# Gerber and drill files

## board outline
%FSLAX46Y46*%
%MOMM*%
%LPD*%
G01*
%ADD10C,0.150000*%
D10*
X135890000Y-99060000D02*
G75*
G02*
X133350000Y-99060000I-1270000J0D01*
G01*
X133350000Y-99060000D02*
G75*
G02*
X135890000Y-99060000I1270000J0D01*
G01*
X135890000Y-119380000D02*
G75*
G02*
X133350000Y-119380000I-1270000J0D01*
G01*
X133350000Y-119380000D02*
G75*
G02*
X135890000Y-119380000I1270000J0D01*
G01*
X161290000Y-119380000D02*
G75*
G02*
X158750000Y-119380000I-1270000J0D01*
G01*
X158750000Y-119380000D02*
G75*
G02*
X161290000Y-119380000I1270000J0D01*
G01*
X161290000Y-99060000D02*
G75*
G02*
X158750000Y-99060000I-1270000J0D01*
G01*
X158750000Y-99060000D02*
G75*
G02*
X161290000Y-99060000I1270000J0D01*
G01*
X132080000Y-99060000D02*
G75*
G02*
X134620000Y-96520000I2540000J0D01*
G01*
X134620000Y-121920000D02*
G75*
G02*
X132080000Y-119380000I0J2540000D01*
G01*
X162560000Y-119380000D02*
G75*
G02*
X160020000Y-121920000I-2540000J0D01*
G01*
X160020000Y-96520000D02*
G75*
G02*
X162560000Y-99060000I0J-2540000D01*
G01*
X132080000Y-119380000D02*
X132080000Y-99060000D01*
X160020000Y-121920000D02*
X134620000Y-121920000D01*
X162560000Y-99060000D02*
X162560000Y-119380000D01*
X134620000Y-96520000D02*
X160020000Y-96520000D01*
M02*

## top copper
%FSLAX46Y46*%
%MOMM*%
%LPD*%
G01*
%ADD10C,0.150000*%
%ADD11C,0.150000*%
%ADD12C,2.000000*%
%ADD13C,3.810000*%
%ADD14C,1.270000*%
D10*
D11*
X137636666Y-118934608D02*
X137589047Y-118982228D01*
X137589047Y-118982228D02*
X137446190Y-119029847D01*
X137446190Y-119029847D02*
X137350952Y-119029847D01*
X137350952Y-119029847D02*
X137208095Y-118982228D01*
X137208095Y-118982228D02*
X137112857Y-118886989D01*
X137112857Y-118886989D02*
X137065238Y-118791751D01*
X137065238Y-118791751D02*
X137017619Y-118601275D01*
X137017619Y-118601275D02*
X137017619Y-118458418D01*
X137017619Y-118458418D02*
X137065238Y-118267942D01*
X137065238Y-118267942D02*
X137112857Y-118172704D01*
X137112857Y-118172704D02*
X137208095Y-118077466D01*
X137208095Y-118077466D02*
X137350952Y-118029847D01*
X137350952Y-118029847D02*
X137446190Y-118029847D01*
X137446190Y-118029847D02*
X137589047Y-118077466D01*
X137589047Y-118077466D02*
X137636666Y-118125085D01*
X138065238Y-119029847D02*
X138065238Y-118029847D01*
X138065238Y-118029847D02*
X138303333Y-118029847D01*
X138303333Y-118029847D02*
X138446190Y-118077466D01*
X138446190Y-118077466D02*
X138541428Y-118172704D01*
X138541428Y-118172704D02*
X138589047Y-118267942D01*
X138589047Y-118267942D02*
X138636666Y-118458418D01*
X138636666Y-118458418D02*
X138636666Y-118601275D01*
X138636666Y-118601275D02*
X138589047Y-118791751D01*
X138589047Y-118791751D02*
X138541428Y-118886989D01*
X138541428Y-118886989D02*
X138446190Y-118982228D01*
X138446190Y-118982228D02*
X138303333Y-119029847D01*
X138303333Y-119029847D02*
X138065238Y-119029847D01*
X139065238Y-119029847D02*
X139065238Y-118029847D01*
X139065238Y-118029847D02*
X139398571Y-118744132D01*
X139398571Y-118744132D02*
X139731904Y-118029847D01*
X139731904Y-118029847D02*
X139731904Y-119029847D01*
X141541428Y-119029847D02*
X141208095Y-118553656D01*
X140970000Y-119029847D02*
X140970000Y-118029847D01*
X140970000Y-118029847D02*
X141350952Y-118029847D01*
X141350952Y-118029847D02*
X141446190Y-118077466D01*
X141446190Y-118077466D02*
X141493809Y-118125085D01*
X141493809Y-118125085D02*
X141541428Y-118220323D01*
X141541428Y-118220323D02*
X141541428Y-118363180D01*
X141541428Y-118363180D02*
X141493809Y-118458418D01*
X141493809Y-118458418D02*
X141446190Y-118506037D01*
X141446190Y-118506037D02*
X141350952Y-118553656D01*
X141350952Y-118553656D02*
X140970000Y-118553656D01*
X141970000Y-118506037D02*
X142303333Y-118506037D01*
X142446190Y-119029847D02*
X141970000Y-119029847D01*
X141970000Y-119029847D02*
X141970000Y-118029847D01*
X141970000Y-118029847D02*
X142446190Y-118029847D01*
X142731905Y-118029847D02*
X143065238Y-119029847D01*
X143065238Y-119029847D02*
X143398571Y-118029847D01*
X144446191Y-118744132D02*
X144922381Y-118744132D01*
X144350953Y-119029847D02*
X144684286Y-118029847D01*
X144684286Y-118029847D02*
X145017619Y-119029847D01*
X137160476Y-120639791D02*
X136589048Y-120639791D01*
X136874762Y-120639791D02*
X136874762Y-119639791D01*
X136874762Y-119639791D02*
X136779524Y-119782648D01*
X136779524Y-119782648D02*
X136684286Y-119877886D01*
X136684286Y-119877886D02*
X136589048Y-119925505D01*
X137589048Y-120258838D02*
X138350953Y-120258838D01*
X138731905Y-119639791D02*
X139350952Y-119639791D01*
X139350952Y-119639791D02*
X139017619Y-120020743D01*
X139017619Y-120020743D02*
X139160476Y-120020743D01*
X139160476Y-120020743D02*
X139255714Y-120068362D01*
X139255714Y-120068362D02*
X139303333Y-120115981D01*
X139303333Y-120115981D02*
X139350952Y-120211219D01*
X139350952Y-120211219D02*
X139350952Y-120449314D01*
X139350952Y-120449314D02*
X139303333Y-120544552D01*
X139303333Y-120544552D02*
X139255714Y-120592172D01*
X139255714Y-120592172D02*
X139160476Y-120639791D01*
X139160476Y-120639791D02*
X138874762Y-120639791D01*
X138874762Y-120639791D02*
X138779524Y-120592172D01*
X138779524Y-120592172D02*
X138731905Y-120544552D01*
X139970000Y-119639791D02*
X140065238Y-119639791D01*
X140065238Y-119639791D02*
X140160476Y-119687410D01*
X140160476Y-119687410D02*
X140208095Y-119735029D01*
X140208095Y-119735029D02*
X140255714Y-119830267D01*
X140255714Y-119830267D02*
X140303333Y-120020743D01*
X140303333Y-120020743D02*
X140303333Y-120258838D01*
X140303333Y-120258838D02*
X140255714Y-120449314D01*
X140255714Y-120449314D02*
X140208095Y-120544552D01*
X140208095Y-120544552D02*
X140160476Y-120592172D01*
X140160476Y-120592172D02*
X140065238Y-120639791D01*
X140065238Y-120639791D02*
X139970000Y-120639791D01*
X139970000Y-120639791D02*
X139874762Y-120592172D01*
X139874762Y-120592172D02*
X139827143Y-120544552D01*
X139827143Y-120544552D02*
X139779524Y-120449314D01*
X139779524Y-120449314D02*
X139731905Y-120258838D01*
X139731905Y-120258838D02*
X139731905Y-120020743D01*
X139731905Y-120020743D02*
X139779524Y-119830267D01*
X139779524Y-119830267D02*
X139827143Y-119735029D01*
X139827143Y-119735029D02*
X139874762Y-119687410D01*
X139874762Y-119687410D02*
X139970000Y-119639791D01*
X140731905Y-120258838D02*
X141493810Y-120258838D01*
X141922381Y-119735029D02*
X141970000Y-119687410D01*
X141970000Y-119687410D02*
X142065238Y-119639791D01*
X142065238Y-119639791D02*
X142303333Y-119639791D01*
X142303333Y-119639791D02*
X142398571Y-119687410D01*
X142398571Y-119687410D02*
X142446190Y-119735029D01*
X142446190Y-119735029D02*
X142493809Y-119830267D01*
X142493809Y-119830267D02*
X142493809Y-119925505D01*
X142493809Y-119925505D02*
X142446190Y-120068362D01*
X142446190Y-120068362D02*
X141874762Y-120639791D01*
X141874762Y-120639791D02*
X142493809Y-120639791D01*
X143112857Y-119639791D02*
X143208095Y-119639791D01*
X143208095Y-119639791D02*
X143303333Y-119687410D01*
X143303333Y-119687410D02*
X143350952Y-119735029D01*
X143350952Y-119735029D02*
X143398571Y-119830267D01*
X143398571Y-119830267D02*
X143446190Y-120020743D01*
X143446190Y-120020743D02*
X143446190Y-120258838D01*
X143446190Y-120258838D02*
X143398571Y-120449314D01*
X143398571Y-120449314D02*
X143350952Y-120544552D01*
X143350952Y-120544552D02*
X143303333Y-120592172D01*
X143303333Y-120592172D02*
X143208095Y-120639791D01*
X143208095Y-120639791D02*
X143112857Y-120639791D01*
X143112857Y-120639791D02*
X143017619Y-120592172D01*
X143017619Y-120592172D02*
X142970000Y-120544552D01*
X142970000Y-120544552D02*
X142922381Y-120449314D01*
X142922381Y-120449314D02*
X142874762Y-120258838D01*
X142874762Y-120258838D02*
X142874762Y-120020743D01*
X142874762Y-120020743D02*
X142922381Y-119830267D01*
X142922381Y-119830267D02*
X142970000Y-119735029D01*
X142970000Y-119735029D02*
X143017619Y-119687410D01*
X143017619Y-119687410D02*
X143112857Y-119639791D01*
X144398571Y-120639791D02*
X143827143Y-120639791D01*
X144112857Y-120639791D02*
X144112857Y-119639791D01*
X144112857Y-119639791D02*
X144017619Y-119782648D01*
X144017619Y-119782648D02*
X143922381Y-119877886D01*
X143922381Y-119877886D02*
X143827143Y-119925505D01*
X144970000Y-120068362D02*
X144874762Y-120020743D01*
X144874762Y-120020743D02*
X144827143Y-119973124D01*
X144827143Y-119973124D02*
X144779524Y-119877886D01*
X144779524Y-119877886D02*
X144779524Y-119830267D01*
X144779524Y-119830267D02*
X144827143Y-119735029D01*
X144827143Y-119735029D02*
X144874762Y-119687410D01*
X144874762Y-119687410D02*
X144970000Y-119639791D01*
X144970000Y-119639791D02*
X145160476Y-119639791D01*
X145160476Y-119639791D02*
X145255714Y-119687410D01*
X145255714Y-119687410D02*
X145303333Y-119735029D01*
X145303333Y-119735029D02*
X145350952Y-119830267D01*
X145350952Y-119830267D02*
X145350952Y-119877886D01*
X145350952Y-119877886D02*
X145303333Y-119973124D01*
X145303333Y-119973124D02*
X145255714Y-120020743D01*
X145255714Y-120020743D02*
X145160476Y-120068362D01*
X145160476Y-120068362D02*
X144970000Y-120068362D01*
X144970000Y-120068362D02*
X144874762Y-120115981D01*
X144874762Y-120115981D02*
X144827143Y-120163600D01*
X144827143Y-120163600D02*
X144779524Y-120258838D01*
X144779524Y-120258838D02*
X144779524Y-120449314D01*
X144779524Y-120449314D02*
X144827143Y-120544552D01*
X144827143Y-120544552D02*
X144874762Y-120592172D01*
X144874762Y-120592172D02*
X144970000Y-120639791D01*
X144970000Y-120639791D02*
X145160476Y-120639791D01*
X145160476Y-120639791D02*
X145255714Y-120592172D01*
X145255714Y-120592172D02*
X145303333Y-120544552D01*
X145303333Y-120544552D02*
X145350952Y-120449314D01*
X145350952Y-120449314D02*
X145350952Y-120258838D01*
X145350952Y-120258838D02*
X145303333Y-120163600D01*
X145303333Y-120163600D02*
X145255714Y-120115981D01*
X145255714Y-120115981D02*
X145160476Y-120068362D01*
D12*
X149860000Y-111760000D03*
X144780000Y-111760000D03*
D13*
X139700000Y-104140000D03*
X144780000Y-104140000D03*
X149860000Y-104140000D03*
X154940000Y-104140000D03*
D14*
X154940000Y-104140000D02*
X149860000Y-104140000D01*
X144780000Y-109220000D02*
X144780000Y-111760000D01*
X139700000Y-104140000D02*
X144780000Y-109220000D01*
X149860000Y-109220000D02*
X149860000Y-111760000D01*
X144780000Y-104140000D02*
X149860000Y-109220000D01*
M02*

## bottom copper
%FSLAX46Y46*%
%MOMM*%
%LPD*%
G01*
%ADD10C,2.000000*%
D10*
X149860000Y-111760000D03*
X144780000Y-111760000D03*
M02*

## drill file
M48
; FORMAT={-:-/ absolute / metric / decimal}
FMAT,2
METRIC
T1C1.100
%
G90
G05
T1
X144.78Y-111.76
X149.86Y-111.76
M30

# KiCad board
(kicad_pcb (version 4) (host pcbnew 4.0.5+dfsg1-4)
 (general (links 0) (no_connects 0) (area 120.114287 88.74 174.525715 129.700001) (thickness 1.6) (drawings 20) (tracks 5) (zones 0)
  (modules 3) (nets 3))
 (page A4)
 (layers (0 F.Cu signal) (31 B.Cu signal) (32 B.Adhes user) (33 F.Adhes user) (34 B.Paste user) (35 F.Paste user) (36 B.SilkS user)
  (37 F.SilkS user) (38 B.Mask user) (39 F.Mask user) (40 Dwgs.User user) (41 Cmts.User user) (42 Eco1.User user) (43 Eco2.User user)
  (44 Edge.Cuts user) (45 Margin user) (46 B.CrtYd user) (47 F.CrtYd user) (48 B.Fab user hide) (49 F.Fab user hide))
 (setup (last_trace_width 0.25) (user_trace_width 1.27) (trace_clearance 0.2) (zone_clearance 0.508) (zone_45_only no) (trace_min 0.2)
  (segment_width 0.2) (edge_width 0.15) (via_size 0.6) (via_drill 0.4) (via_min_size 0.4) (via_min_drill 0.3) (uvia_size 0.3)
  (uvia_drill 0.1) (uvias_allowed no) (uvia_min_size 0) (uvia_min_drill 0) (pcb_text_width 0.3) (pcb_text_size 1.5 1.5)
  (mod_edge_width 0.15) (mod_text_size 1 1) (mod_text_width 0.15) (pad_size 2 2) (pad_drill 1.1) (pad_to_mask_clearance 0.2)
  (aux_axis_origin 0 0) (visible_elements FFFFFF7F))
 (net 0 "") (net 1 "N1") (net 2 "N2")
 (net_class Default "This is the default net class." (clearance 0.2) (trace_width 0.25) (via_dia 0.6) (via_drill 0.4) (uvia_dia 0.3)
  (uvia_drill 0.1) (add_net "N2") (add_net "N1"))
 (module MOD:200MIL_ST (layer F.Cu) (at 147.32 115.57 180)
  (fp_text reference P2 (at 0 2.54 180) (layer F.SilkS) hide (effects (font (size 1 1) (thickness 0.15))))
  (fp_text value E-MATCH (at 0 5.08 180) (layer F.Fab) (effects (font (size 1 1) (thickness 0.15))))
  (pad 1 thru_hole circle (at -2.54 3.81 180) (size 2 2) (drill 1.1) (layers *.Cu *.Mask) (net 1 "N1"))
  (pad 2 thru_hole circle (at 2.54 3.81 180) (size 2 2) (drill 1.1) (layers *.Cu *.Mask) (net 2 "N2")))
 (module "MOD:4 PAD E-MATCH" (layer F.Cu) (at 147.32 104.14)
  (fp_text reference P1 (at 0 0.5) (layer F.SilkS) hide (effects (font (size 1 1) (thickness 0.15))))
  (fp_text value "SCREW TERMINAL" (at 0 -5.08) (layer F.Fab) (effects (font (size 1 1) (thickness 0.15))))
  (pad 1 connect circle (at -7.62 0) (size 3.81 3.81) (layers F.Cu F.Mask) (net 2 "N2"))
  (pad 2 connect circle (at -2.54 0) (size 3.81 3.81) (layers F.Cu F.Mask) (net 1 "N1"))
  (pad 3 connect circle (at 2.54 0) (size 3.81 3.81) (layers F.Cu F.Mask))
  (pad 4 connect circle (at 7.62 0) (size 3.81 3.81) (layers F.Cu F.Mask)))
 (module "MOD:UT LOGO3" (layer F.Cu) (at 137.16 110.49)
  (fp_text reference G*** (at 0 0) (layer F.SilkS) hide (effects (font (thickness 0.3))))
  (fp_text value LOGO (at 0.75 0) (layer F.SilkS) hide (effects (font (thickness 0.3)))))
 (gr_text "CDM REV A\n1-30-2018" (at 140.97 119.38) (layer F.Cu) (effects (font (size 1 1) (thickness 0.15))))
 (gr_circle (center 134.62 99.06) (end 134.62 97.79) (layer Edge.Cuts) (width 0.15))
 (gr_circle (center 134.62 119.38) (end 134.62 118.11) (layer Edge.Cuts) (width 0.15))
 (gr_circle (center 160.02 119.38) (end 160.02 118.11) (layer Edge.Cuts) (width 0.15))
 (gr_circle (center 160.02 99.06) (end 160.02 97.79) (layer Edge.Cuts) (width 0.15))
 (gr_arc (start 134.62 99.06) (end 132.08 99.06) (angle 90) (layer Edge.Cuts) (width 0.15))
 (gr_arc (start 134.62 119.38) (end 134.62 121.92) (angle 90) (layer Edge.Cuts) (width 0.15))
 (gr_arc (start 160.02 119.38) (end 162.56 119.38) (angle 90) (layer Edge.Cuts) (width 0.15))
 (gr_arc (start 160.02 99.06) (end 160.02 96.52) (angle 90) (layer Edge.Cuts) (width 0.15))
 (gr_line (start 132.08 119.38) (end 132.08 99.06) (layer Edge.Cuts) (width 0.15))
 (gr_line (start 160.02 121.92) (end 134.62 121.92) (layer Edge.Cuts) (width 0.15))
 (gr_line (start 162.56 99.06) (end 162.56 119.38) (layer Edge.Cuts) (width 0.15))
 (gr_line (start 134.62 96.52) (end 160.02 96.52) (layer Edge.Cuts) (width 0.15))
 (segment (start 154.94 104.14) (end 149.86 104.14) (width 1.27) (layer F.Cu) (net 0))
 (segment (start 144.78 109.22) (end 144.78 111.76) (width 1.27) (layer F.Cu) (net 2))
 (segment (start 139.7 104.14) (end 144.78 109.22) (width 1.27) (layer F.Cu) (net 2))
 (segment (start 149.86 109.22) (end 149.86 111.76) (width 1.27) (layer F.Cu) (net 1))
 (segment (start 144.78 104.14) (end 149.86 109.22) (width 1.27) (layer F.Cu) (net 1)))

